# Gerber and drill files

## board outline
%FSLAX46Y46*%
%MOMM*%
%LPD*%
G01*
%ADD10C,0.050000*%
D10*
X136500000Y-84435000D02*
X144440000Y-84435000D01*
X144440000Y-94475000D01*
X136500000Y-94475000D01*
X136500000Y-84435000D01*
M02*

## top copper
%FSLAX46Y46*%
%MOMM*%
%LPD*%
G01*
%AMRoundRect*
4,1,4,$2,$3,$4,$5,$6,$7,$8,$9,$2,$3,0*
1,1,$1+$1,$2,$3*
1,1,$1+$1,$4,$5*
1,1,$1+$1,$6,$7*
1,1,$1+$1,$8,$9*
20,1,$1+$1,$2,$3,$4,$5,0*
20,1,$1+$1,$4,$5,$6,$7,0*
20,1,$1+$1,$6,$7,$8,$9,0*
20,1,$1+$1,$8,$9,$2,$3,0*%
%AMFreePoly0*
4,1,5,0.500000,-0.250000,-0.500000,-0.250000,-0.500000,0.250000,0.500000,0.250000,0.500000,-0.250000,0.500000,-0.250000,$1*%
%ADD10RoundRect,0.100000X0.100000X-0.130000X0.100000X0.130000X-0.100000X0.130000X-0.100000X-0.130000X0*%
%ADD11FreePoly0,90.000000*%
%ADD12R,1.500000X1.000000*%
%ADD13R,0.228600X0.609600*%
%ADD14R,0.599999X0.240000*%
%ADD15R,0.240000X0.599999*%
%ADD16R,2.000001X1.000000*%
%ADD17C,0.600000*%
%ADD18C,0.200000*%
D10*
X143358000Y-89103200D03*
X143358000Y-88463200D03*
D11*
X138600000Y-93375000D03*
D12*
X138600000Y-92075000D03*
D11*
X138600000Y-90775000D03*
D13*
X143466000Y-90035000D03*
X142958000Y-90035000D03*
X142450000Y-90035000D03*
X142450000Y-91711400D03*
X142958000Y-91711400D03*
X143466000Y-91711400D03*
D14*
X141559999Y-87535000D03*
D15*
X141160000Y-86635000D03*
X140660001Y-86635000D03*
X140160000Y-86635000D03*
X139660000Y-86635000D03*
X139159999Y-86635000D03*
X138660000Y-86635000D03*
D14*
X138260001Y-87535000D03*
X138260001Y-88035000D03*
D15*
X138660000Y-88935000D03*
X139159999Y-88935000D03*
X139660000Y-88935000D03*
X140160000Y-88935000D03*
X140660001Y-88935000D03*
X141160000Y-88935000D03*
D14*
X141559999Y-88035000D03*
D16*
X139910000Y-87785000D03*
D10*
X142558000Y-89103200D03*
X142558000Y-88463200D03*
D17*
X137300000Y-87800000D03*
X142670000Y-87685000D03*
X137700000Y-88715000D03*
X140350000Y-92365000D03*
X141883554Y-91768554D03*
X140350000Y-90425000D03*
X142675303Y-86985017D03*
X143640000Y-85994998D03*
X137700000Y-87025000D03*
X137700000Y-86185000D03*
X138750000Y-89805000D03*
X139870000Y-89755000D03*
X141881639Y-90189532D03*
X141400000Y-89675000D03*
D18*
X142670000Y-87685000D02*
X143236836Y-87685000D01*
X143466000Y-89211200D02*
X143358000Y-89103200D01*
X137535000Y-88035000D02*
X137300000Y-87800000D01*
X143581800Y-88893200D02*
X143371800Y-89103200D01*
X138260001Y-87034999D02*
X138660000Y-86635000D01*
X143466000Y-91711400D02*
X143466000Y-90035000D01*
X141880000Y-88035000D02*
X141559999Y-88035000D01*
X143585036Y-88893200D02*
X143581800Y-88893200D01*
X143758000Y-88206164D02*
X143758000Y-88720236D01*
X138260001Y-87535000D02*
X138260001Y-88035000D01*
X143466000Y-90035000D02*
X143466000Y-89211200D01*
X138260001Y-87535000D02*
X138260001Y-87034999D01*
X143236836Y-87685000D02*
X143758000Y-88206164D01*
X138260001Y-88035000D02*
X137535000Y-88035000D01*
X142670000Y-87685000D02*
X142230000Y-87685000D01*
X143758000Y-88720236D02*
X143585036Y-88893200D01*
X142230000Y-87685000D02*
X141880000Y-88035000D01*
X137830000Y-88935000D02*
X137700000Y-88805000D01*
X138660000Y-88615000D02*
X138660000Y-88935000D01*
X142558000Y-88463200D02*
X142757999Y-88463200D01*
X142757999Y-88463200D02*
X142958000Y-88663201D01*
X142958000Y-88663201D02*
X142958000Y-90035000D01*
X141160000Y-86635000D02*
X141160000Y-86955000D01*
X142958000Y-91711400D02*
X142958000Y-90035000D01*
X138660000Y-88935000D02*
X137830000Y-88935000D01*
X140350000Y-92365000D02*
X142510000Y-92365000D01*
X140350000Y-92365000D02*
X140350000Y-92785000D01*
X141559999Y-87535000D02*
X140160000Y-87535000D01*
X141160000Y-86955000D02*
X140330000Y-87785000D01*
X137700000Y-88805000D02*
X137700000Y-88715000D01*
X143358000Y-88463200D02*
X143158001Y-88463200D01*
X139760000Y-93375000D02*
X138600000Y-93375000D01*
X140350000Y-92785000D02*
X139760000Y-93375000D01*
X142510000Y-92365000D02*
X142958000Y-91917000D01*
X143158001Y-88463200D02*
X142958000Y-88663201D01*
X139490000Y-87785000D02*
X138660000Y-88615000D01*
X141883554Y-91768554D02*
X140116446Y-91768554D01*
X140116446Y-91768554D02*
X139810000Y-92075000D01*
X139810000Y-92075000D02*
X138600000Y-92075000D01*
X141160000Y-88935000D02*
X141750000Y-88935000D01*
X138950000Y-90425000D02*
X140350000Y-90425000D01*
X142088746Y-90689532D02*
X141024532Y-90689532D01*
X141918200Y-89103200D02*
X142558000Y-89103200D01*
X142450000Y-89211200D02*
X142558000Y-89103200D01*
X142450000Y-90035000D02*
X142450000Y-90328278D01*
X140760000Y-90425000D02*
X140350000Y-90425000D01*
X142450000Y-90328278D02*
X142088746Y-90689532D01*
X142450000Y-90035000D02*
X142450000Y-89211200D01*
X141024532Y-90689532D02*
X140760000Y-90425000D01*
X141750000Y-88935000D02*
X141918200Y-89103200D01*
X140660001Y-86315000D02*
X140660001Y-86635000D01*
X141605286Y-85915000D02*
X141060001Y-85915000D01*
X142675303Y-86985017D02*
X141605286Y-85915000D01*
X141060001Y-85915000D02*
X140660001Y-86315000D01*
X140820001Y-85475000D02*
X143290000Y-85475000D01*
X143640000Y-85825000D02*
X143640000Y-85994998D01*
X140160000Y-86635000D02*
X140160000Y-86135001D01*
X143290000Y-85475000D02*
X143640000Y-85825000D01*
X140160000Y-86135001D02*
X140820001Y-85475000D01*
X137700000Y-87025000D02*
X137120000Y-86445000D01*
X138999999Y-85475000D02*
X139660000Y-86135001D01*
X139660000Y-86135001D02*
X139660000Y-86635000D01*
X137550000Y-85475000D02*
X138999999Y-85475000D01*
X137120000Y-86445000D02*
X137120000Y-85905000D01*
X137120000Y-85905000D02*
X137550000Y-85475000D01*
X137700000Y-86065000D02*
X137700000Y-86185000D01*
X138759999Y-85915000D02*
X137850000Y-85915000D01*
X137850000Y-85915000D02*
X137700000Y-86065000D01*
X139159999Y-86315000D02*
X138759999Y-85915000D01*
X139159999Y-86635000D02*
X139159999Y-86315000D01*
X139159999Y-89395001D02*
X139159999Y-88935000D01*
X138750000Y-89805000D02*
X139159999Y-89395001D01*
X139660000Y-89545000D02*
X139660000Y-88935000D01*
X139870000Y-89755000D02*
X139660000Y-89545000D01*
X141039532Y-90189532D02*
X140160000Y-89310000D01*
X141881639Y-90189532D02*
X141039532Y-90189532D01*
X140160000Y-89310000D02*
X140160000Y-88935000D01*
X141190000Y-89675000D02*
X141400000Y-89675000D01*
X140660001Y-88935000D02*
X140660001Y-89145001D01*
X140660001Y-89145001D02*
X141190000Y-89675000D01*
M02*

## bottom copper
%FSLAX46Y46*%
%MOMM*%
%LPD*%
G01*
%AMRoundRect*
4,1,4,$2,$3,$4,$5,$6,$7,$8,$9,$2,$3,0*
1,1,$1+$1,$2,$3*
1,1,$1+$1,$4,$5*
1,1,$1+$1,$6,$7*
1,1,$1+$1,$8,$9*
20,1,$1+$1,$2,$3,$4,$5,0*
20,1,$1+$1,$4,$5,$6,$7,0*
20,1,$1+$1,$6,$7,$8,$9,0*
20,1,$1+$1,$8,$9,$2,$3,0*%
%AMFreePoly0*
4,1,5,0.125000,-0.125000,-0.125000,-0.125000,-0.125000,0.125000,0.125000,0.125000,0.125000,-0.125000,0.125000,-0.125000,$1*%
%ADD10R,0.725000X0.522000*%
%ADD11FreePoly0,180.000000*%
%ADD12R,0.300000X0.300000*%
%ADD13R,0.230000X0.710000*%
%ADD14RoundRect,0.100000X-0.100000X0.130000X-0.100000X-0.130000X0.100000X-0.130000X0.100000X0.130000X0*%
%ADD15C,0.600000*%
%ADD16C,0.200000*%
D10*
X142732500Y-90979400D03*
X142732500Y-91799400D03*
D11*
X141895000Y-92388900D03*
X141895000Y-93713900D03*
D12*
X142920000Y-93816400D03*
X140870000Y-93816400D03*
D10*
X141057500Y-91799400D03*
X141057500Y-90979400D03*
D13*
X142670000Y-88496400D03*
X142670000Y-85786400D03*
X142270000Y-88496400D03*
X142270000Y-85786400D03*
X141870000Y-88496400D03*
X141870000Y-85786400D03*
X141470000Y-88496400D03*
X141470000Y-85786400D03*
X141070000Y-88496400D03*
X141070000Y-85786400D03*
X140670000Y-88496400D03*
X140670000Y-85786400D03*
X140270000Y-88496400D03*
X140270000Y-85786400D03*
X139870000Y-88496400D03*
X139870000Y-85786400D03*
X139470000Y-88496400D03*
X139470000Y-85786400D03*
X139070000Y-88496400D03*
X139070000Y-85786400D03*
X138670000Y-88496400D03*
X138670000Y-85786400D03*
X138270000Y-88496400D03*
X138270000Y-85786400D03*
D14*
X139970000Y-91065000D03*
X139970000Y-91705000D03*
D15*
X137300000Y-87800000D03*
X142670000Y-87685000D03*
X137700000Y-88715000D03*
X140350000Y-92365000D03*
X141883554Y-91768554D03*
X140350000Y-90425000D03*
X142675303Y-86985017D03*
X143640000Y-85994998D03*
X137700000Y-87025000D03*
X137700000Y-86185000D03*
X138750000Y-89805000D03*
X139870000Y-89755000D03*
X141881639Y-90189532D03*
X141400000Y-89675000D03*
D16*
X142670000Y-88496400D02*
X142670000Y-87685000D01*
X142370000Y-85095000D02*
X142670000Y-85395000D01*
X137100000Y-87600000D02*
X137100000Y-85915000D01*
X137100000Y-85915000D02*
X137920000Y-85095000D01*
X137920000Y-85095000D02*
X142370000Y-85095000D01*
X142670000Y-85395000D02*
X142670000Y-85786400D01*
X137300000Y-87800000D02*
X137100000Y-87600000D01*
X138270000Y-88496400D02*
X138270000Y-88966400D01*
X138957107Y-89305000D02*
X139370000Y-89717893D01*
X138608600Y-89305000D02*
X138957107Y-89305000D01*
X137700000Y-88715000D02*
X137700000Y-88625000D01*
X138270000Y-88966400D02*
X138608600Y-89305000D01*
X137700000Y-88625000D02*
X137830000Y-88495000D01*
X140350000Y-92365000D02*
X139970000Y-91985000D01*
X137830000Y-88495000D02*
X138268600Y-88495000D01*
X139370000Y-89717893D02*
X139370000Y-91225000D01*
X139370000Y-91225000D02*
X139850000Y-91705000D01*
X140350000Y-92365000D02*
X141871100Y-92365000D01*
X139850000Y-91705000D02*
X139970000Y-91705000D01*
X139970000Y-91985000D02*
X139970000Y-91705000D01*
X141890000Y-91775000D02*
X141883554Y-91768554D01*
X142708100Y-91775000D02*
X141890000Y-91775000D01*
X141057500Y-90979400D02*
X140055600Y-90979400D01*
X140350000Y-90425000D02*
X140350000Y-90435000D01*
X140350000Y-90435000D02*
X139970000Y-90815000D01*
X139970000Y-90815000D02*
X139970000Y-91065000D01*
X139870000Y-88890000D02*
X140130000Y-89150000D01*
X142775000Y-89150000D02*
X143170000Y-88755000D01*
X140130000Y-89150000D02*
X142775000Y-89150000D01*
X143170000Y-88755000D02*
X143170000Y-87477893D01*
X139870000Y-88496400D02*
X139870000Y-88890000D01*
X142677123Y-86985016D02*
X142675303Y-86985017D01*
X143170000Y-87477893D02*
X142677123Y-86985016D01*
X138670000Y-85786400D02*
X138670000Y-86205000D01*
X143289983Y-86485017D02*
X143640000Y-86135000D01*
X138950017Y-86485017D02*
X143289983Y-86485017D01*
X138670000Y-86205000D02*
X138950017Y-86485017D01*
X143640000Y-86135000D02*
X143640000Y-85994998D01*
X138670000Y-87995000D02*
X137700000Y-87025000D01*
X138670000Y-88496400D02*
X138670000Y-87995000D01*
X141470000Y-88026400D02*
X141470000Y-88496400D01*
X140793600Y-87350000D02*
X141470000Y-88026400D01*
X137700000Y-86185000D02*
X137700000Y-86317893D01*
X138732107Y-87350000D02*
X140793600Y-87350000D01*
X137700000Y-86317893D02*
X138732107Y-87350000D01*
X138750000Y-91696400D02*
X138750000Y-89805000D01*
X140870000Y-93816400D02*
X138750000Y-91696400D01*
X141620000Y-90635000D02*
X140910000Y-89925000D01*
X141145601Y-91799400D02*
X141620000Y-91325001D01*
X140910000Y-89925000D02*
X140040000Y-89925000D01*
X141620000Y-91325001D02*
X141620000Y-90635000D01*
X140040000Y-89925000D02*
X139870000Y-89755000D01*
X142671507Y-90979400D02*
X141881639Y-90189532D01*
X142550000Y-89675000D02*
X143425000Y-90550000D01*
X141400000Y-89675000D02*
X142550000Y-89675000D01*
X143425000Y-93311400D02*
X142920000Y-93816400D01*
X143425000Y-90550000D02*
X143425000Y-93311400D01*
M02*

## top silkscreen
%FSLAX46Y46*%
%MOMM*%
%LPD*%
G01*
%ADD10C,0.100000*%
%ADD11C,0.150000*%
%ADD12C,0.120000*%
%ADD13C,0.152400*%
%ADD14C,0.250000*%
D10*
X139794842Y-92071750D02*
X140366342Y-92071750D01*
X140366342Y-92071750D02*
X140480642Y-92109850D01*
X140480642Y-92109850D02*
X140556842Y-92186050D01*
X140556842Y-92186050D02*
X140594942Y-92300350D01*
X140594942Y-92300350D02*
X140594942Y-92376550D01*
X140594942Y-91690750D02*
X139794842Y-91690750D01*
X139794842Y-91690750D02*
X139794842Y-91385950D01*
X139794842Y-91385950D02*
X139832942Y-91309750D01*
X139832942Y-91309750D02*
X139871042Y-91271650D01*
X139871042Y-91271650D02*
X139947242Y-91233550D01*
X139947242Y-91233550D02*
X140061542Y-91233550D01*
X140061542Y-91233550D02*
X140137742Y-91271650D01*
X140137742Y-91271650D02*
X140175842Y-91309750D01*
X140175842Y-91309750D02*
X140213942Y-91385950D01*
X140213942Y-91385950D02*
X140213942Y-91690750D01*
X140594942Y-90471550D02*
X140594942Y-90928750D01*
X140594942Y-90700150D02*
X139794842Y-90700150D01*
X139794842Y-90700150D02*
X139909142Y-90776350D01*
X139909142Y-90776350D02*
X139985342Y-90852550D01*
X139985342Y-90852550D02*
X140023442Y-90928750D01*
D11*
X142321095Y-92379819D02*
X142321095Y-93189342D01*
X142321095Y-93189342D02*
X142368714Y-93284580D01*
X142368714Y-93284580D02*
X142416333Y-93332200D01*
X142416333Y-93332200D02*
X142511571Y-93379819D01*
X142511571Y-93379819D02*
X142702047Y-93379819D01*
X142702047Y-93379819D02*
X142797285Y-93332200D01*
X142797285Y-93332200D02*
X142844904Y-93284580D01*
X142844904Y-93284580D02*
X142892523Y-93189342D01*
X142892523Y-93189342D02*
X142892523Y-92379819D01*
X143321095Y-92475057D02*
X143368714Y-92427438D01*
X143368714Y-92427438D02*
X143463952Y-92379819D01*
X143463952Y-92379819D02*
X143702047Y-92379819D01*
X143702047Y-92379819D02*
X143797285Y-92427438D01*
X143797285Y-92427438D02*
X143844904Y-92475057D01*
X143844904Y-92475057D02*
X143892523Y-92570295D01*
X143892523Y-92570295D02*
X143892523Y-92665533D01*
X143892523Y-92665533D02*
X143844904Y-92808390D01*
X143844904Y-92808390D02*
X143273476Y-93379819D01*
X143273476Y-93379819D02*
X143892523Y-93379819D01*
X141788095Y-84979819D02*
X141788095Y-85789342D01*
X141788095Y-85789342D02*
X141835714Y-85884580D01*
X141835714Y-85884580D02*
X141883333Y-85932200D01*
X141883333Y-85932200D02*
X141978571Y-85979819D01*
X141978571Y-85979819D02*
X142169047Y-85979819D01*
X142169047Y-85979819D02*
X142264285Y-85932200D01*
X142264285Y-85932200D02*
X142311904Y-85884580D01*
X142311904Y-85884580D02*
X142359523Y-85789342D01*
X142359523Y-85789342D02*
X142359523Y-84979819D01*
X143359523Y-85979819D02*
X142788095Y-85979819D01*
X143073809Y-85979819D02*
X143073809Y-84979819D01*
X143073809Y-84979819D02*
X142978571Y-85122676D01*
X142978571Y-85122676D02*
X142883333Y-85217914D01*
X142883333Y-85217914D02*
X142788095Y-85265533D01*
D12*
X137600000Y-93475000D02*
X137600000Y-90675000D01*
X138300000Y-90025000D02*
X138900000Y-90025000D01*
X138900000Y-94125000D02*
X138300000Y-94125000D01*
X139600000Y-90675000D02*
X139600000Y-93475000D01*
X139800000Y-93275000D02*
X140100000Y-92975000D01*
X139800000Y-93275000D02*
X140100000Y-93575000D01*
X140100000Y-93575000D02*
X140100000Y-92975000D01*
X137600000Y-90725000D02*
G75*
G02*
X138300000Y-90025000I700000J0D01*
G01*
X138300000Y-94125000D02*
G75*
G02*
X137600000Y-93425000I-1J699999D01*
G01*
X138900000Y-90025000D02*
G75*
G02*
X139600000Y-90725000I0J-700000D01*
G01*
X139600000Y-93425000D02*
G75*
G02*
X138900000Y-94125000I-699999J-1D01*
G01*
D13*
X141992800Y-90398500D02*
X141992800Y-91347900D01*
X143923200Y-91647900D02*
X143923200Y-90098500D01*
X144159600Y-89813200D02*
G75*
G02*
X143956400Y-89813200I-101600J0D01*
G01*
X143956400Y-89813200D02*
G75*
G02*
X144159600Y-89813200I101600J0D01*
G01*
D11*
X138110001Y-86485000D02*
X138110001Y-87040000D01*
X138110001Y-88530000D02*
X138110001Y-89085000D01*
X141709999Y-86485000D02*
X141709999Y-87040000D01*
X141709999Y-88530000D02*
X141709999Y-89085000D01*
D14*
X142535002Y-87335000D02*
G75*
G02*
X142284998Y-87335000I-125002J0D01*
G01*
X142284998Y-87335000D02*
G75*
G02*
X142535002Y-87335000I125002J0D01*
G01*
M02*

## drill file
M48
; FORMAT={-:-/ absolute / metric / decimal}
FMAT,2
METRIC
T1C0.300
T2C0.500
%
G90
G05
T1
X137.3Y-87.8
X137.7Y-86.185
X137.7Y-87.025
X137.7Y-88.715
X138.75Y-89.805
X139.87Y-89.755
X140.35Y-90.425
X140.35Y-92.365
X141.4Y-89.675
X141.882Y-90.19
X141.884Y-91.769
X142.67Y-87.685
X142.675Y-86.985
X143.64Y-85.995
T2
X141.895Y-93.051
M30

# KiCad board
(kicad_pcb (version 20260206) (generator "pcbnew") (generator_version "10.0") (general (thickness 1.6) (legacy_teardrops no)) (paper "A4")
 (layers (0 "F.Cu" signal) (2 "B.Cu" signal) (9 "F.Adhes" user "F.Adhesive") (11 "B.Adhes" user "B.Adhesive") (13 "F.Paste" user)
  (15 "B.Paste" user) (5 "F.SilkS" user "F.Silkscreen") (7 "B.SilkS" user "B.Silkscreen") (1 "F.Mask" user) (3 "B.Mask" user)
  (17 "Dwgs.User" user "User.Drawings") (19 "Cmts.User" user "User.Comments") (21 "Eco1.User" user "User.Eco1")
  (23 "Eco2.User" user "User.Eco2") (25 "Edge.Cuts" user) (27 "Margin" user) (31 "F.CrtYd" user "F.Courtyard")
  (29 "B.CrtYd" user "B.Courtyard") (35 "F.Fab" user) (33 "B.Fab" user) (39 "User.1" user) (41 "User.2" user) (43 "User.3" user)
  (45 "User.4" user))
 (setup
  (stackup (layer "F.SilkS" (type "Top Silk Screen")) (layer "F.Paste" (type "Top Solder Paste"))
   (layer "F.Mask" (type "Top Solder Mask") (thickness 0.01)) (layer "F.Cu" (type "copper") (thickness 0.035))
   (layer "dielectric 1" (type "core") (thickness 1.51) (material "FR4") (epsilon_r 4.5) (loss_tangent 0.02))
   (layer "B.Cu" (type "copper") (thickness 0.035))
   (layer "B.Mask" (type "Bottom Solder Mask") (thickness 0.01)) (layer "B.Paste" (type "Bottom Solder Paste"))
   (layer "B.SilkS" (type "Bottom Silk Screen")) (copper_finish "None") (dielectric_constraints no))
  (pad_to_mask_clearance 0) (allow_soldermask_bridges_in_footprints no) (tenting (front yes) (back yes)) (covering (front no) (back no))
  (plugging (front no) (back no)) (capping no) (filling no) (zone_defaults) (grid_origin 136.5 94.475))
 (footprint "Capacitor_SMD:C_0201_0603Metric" (layer "F.Cu") (at 143.358 88.7832 90)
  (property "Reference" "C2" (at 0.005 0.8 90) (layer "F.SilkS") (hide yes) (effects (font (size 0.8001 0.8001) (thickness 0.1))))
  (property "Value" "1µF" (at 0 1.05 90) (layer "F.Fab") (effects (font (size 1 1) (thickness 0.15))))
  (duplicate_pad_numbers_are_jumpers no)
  (pad "" smd roundrect (at -0.345 0 90) (size 0.318 0.36) (layers "F.Paste") (roundrect_rratio 0.25))
  (pad "" smd roundrect (at 0.345 0 90) (size 0.318 0.36) (layers "F.Paste") (roundrect_rratio 0.25))
  (pad "1" smd roundrect (at -0.32 0 90) (size 0.46 0.4) (layers "F.Cu" "F.Mask") (roundrect_rratio 0.25) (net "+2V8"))
  (pad "2" smd roundrect (at 0.32 0 90) (size 0.46 0.4) (layers "F.Cu" "F.Mask") (roundrect_rratio 0.25) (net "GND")))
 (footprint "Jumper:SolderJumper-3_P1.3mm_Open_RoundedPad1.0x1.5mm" (layer "F.Cu") (at 138.6 92.075 90)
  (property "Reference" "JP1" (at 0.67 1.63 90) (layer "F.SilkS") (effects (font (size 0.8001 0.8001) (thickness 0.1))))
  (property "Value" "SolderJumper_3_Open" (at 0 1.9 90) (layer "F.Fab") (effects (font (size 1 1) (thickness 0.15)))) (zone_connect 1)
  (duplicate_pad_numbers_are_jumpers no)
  (fp_line (start -1.4 -1) (end 1.4 -1) (stroke (width 0.12) (type solid)) (layer "F.SilkS"))
  (fp_line (start 2.05 -0.3) (end 2.05 0.3) (stroke (width 0.12) (type solid)) (layer "F.SilkS"))
  (fp_line (start -2.05 0.3) (end -2.05 -0.3) (stroke (width 0.12) (type solid)) (layer "F.SilkS"))
  (fp_line (start 1.4 1) (end -1.4 1) (stroke (width 0.12) (type solid)) (layer "F.SilkS"))
  (fp_line (start -1.2 1.2) (end -0.9 1.5) (stroke (width 0.12) (type solid)) (layer "F.SilkS"))
  (fp_line (start -1.2 1.2) (end -1.5 1.5) (stroke (width 0.12) (type solid)) (layer "F.SilkS"))
  (fp_line (start -1.5 1.5) (end -0.9 1.5) (stroke (width 0.12) (type solid)) (layer "F.SilkS"))
  (fp_arc (start 1.35 -1) (mid 1.844975 -0.794975) (end 2.05 -0.3) (stroke (width 0.12) (type solid)) (layer "F.SilkS"))
  (fp_arc (start -2.05 -0.3) (mid -1.844975 -0.794975) (end -1.35 -1) (stroke (width 0.12) (type solid)) (layer "F.SilkS"))
  (fp_arc (start 2.05 0.3) (mid 1.844975 0.794975) (end 1.35 1) (stroke (width 0.12) (type solid)) (layer "F.SilkS"))
  (fp_arc (start -1.35 1) (mid -1.844975 0.794975) (end -2.05 0.3) (stroke (width 0.12) (type solid)) (layer "F.SilkS"))
  (pad "1" smd custom (at -1.3 0 90) (size 1 0.5) (layers "F.Cu" "F.Mask") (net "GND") (zone_connect 2) (thermal_bridge_angle 45)
   (options (clearance outline) (anchor rect)) (primitives))
  (pad "2" smd rect (at 0 0 90) (size 1 1.5) (layers "F.Cu" "F.Mask") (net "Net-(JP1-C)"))
  (pad "3" smd custom (at 1.3 0 90) (size 1 0.5) (layers "F.Cu" "F.Mask") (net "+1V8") (zone_connect 2) (thermal_bridge_angle 45)
   (options (clearance outline) (anchor rect)) (primitives)))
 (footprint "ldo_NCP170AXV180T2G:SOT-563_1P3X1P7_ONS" (layer "F.Cu") (at 142.958 90.8732 -90)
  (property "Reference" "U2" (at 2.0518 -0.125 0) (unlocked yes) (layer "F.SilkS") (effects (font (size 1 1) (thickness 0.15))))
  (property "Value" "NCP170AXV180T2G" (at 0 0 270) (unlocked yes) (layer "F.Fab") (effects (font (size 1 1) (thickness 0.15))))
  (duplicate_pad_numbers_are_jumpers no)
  (fp_line (start -0.4747 0.9652) (end 0.4747 0.9652) (stroke (width 0.1524) (type solid)) (layer "F.SilkS"))
  (fp_line (start 0.7747 -0.9652) (end -0.7747 -0.9652) (stroke (width 0.1524) (type solid)) (layer "F.SilkS"))
  (fp_circle (center -1.06 -1.1) (end -0.9584 -1.1) (stroke (width 0.1524) (type solid)) (fill no) (layer "F.SilkS"))
  (pad "1" smd rect (at -0.8382 -0.508 270) (size 0.6096 0.2286) (layers "F.Cu" "F.Mask" "F.Paste") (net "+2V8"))
  (pad "2" smd rect (at -0.8382 0 270) (size 0.6096 0.2286) (layers "F.Cu" "F.Mask" "F.Paste") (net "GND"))
  (pad "3" smd rect (at -0.8382 0.508 270) (size 0.6096 0.2286) (layers "F.Cu" "F.Mask" "F.Paste") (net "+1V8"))
  (pad "4" smd rect (at 0.8382 0.508 270) (size 0.6096 0.2286) (layers "F.Cu" "F.Mask" "F.Paste") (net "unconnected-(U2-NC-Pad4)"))
  (pad "5" smd rect (at 0.8382 0 270) (size 0.6096 0.2286) (layers "F.Cu" "F.Mask" "F.Paste") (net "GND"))
  (pad "6" smd rect (at 0.8382 -0.508 270) (size 0.6096 0.2286) (layers "F.Cu" "F.Mask" "F.Paste") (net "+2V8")))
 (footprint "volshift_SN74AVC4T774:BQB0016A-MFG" (layer "F.Cu") (at 139.91 87.785 -90)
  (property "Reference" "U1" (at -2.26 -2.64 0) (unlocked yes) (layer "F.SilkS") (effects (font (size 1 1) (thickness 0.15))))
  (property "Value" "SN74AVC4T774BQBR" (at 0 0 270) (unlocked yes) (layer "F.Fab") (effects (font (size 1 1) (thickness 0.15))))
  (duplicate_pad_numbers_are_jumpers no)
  (fp_line (start -1.3 1.799999) (end -0.745 1.799999) (stroke (width 0.15) (type solid)) (layer "F.SilkS"))
  (fp_line (start 0.745 1.799999) (end 1.3 1.799999) (stroke (width 0.15) (type solid)) (layer "F.SilkS"))
  (fp_line (start -1.3 -1.799999) (end -0.745 -1.799999) (stroke (width 0.15) (type solid)) (layer "F.SilkS"))
  (fp_line (start 0.745 -1.799999) (end 1.3 -1.799999) (stroke (width 0.15) (type solid)) (layer "F.SilkS"))
  (fp_circle (center -0.45 -2.5) (end -0.324998 -2.5) (stroke (width 0.25) (type solid)) (fill no) (layer "F.SilkS"))
  (pad "1" smd rect (at -0.25 -1.649999 270) (size 0.24 0.599999) (layers "F.Cu" "F.Mask" "F.Paste") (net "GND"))
  (pad "2" smd rect (at -1.15 -1.25) (size 0.24 0.599999) (layers "F.Cu" "F.Mask" "F.Paste") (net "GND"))
  (pad "3" smd rect (at -1.15 -0.750001) (size 0.24 0.599999) (layers "F.Cu" "F.Mask" "F.Paste") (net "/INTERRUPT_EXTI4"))
  (pad "4" smd rect (at -1.15 -0.25) (size 0.24 0.599999) (layers "F.Cu" "F.Mask" "F.Paste") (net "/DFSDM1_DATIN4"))
  (pad "5" smd rect (at -1.15 0.25) (size 0.24 0.599999) (layers "F.Cu" "F.Mask" "F.Paste") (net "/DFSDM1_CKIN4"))
  (pad "6" smd rect (at -1.15 0.750001) (size 0.24 0.599999) (layers "F.Cu" "F.Mask" "F.Paste") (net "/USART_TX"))
  (pad "7" smd rect (at -1.15 1.25) (size 0.24 0.599999) (layers "F.Cu" "F.Mask" "F.Paste") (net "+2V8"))
  (pad "8" smd rect (at -0.25 1.649999 270) (size 0.24 0.599999) (layers "F.Cu" "F.Mask" "F.Paste") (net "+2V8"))
  (pad "9" smd rect (at 0.25 1.649999 270) (size 0.24 0.599999) (layers "F.Cu" "F.Mask" "F.Paste") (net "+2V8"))
  (pad "10" smd rect (at 1.15 1.25) (size 0.24 0.599999) (layers "F.Cu" "F.Mask" "F.Paste") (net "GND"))
  (pad "11" smd rect (at 1.15 0.750001) (size 0.24 0.599999) (layers "F.Cu" "F.Mask" "F.Paste") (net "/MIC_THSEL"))
  (pad "12" smd rect (at 1.15 0.25) (size 0.24 0.599999) (layers "F.Cu" "F.Mask" "F.Paste") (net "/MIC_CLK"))
  (pad "13" smd rect (at 1.15 -0.25) (size 0.24 0.599999) (layers "F.Cu" "F.Mask" "F.Paste") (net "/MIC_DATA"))
  (pad "14" smd rect (at 1.15 -0.750001) (size 0.24 0.599999) (layers "F.Cu" "F.Mask" "F.Paste") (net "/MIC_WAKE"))
  (pad "15" smd rect (at 1.15 -1.25) (size 0.24 0.599999) (layers "F.Cu" "F.Mask" "F.Paste") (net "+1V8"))
  (pad "16" smd rect (at 0.25 -1.649999 270) (size 0.24 0.599999) (layers "F.Cu" "F.Mask" "F.Paste") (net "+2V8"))
  (pad "17" smd rect (at 0 0 270) (size 1 2.000001) (layers "F.Cu" "F.Mask") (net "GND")))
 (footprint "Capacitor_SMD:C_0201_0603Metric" (layer "F.Cu") (at 142.558 88.7832 90)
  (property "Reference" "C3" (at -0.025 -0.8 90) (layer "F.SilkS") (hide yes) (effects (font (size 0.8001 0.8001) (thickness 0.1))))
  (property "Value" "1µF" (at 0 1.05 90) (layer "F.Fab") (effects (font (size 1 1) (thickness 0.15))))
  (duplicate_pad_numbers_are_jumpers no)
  (pad "" smd roundrect (at -0.345 0 90) (size 0.318 0.36) (layers "F.Paste") (roundrect_rratio 0.25))
  (pad "" smd roundrect (at 0.345 0 90) (size 0.318 0.36) (layers "F.Paste") (roundrect_rratio 0.25))
  (pad "1" smd roundrect (at -0.32 0 90) (size 0.46 0.4) (layers "F.Cu" "F.Mask") (roundrect_rratio 0.25) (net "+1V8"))
  (pad "2" smd roundrect (at 0.32 0 90) (size 0.46 0.4) (layers "F.Cu" "F.Mask") (roundrect_rratio 0.25) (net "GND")))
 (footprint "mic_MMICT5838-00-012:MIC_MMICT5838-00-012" (layer "B.Cu") (at 141.895 92.3414 180)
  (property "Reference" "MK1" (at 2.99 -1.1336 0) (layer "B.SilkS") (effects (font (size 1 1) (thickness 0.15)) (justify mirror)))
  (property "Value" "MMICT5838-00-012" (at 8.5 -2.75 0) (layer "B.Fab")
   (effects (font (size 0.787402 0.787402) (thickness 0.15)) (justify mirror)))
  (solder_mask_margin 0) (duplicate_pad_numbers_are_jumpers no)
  (pad "" np_thru_hole circle (at 0 -0.71 180) (size 0.5 0.5) (drill 0.5) (layers "*.Cu" "*.Mask"))
  (pad "1" smd rect (at -0.8375 1.362 180) (size 0.725 0.522) (layers "B.Cu") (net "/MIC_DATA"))
  (pad "2" smd rect (at -0.8375 0.542 180) (size 0.725 0.522) (layers "B.Cu") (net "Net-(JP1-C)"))
  (pad "3_1" smd custom (at 0 -0.0475 180) (size 0.25 0.25) (layers "B.Cu") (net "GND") (options (clearance outline) (anchor rect))
   (primitives))
  (pad "3_2" smd custom (at 0 -1.3725 180) (size 0.25 0.25) (layers "B.Cu") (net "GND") (options (clearance outline) (anchor rect))
   (primitives))
  (pad "4" smd rect (at -1.025 -1.475 180) (size 0.3 0.3) (layers "B.Cu") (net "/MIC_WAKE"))
  (pad "5" smd rect (at 1.025 -1.475 180) (size 0.3 0.3) (layers "B.Cu") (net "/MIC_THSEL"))
  (pad "6" smd rect (at 0.8375 0.542 180) (size 0.725 0.522) (layers "B.Cu") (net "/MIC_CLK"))
  (pad "7" smd rect (at 0.8375 1.362 180) (size 0.725 0.522) (layers "B.Cu") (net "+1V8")))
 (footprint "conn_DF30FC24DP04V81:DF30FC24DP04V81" (layer "B.Cu") (at 140.47 87.1414 180)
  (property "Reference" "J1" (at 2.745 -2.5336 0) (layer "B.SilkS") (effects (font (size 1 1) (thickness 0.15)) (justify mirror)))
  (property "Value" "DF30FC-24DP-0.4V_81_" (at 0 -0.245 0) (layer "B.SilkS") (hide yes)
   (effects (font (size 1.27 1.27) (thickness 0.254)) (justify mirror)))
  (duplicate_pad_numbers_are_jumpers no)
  (pad "1" smd rect (at -2.2 -1.355 180) (size 0.23 0.71) (layers "B.Cu" "B.Mask" "B.Paste") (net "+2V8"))
  (pad "2" smd rect (at -2.2 1.355 180) (size 0.23 0.71) (layers "B.Cu" "B.Mask" "B.Paste") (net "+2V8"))
  (pad "3" smd rect (at -1.8 -1.355 180) (size 0.23 0.71) (layers "B.Cu" "B.Mask" "B.Paste") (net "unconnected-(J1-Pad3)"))
  (pad "4" smd rect (at -1.8 1.355 180) (size 0.23 0.71) (layers "B.Cu" "B.Mask" "B.Paste") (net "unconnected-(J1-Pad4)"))
  (pad "5" smd rect (at -1.4 -1.355 180) (size 0.23 0.71) (layers "B.Cu" "B.Mask" "B.Paste") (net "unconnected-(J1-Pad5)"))
  (pad "6" smd rect (at -1.4 1.355 180) (size 0.23 0.71) (layers "B.Cu" "B.Mask" "B.Paste") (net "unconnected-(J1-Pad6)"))
  (pad "7" smd rect (at -1 -1.355 180) (size 0.23 0.71) (layers "B.Cu" "B.Mask" "B.Paste") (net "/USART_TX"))
  (pad "8" smd rect (at -1 1.355 180) (size 0.23 0.71) (layers "B.Cu" "B.Mask" "B.Paste") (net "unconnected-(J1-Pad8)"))
  (pad "9" smd rect (at -0.6 -1.355 180) (size 0.23 0.71) (layers "B.Cu" "B.Mask" "B.Paste") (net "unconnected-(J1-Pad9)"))
  (pad "10" smd rect (at -0.6 1.355 180) (size 0.23 0.71) (layers "B.Cu" "B.Mask" "B.Paste") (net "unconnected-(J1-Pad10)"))
  (pad "11" smd rect (at -0.2 -1.355 180) (size 0.23 0.71) (layers "B.Cu" "B.Mask" "B.Paste") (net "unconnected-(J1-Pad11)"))
  (pad "12" smd rect (at -0.2 1.355 180) (size 0.23 0.71) (layers "B.Cu" "B.Mask" "B.Paste") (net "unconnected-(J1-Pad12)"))
  (pad "13" smd rect (at 0.2 -1.355 180) (size 0.23 0.71) (layers "B.Cu" "B.Mask" "B.Paste") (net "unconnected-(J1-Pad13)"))
  (pad "14" smd rect (at 0.2 1.355 180) (size 0.23 0.71) (layers "B.Cu" "B.Mask" "B.Paste") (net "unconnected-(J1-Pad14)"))
  (pad "15" smd rect (at 0.6 -1.355 180) (size 0.23 0.71) (layers "B.Cu" "B.Mask" "B.Paste") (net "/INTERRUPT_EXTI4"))
  (pad "16" smd rect (at 0.6 1.355 180) (size 0.23 0.71) (layers "B.Cu" "B.Mask" "B.Paste") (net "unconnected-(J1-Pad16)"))
  (pad "17" smd rect (at 1 -1.355 180) (size 0.23 0.71) (layers "B.Cu" "B.Mask" "B.Paste") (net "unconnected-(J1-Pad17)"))
  (pad "18" smd rect (at 1 1.355 180) (size 0.23 0.71) (layers "B.Cu" "B.Mask" "B.Paste") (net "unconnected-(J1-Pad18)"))
  (pad "19" smd rect (at 1.4 -1.355 180) (size 0.23 0.71) (layers "B.Cu" "B.Mask" "B.Paste") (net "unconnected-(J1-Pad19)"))
  (pad "20" smd rect (at 1.4 1.355 180) (size 0.23 0.71) (layers "B.Cu" "B.Mask" "B.Paste") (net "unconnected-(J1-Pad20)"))
  (pad "21" smd rect (at 1.8 -1.355 180) (size 0.23 0.71) (layers "B.Cu" "B.Mask" "B.Paste") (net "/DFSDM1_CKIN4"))
  (pad "22" smd rect (at 1.8 1.355 180) (size 0.23 0.71) (layers "B.Cu" "B.Mask" "B.Paste") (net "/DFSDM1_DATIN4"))
  (pad "23" smd rect (at 2.2 -1.355 180) (size 0.23 0.71) (layers "B.Cu" "B.Mask" "B.Paste") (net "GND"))
  (pad "24" smd rect (at 2.2 1.355 180) (size 0.23 0.71) (layers "B.Cu" "B.Mask" "B.Paste") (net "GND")))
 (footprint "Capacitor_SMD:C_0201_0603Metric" (layer "B.Cu") (at 139.97 91.385 -90)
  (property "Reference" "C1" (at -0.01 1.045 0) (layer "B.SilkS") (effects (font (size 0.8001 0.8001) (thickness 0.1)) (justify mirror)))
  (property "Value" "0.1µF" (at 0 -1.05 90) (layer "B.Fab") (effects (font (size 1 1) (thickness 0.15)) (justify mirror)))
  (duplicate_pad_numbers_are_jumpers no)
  (pad "" smd roundrect (at -0.345 0 270) (size 0.318 0.36) (layers "B.Paste") (roundrect_rratio 0.25))
  (pad "" smd roundrect (at 0.345 0 270) (size 0.318 0.36) (layers "B.Paste") (roundrect_rratio 0.25))
  (pad "1" smd roundrect (at -0.32 0 270) (size 0.46 0.4) (layers "B.Cu" "B.Mask") (roundrect_rratio 0.25) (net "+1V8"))
  (pad "2" smd roundrect (at 0.32 0 270) (size 0.46 0.4) (layers "B.Cu" "B.Mask") (roundrect_rratio 0.25) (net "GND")))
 (gr_rect (start 136.5 84.435) (end 144.44 94.475) (stroke (width 0.05) (type default)) (fill no) (layer "Edge.Cuts"))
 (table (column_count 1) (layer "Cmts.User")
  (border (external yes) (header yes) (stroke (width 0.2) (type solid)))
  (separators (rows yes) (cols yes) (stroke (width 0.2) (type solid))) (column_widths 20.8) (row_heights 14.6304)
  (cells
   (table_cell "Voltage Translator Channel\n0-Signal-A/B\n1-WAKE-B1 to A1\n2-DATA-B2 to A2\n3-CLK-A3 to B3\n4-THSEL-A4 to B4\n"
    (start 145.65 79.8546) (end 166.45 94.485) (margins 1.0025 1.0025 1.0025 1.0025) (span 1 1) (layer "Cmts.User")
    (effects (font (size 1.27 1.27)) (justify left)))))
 (segment (start 142.67 87.685) (end 143.236836 87.685) (width 0.2) (layer "F.Cu") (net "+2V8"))
 (segment (start 143.466 89.2112) (end 143.358 89.1032) (width 0.2) (layer "F.Cu") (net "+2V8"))
 (segment (start 137.535 88.035) (end 137.3 87.8) (width 0.2) (layer "F.Cu") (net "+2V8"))
 (segment (start 143.5818 88.8932) (end 143.3718 89.1032) (width 0.2) (layer "F.Cu") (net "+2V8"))
 (segment (start 138.260001 87.034999) (end 138.66 86.635) (width 0.2) (layer "F.Cu") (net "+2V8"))
 (segment (start 143.466 91.7114) (end 143.466 90.035) (width 0.2) (layer "F.Cu") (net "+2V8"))
 (segment (start 141.88 88.035) (end 141.559999 88.035) (width 0.2) (layer "F.Cu") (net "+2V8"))
 (segment (start 143.585036 88.8932) (end 143.5818 88.8932) (width 0.2) (layer "F.Cu") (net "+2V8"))
 (segment (start 143.758 88.206164) (end 143.758 88.720236) (width 0.2) (layer "F.Cu") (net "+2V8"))
 (segment (start 138.260001 87.535) (end 138.260001 88.035) (width 0.2) (layer "F.Cu") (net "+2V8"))
 (segment (start 143.466 90.035) (end 143.466 89.2112) (width 0.2) (layer "F.Cu") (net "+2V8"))
 (segment (start 138.260001 87.535) (end 138.260001 87.034999) (width 0.2) (layer "F.Cu") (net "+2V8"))
 (segment (start 143.236836 87.685) (end 143.758 88.206164) (width 0.2) (layer "F.Cu") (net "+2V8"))
 (segment (start 138.260001 88.035) (end 137.535 88.035) (width 0.2) (layer "F.Cu") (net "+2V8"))
 (segment (start 142.67 87.685) (end 142.23 87.685) (width 0.2) (layer "F.Cu") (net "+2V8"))
 (segment (start 143.758 88.720236) (end 143.585036 88.8932) (width 0.2) (layer "F.Cu") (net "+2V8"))
 (segment (start 142.23 87.685) (end 141.88 88.035) (width 0.2) (layer "F.Cu") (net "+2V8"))
 (via (at 137.3 87.8) (size 0.6) (drill 0.3) (layers "F.Cu" "B.Cu") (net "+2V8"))
 (via (at 142.67 87.685) (size 0.6) (drill 0.3) (layers "F.Cu" "B.Cu") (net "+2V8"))
 (segment (start 142.67 88.4964) (end 142.67 87.685) (width 0.2) (layer "B.Cu") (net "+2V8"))
 (segment (start 142.37 85.095) (end 142.67 85.395) (width 0.2) (layer "B.Cu") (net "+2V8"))
 (segment (start 137.1 87.6) (end 137.1 85.915) (width 0.2) (layer "B.Cu") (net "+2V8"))
 (segment (start 137.1 85.915) (end 137.92 85.095) (width 0.2) (layer "B.Cu") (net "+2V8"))
 (segment (start 137.92 85.095) (end 142.37 85.095) (width 0.2) (layer "B.Cu") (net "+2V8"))
 (segment (start 142.67 85.395) (end 142.67 85.7864) (width 0.2) (layer "B.Cu") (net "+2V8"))
 (segment (start 137.3 87.8) (end 137.1 87.6) (width 0.2) (layer "B.Cu") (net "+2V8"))
 (segment (start 137.83 88.935) (end 137.7 88.805) (width 0.2) (layer "F.Cu") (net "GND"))
 (segment (start 138.66 88.615) (end 138.66 88.935) (width 0.2) (layer "F.Cu") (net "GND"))
 (segment (start 142.558 88.4632) (end 142.757999 88.4632) (width 0.2) (layer "F.Cu") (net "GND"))
 (segment (start 142.757999 88.4632) (end 142.958 88.663201) (width 0.2) (layer "F.Cu") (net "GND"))
 (segment (start 142.958 88.663201) (end 142.958 90.035) (width 0.2) (layer "F.Cu") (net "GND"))
 (segment (start 141.16 86.635) (end 141.16 86.955) (width 0.2) (layer "F.Cu") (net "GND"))
 (segment (start 142.958 91.7114) (end 142.958 90.035) (width 0.2) (layer "F.Cu") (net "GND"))
 (segment (start 138.66 88.935) (end 137.83 88.935) (width 0.2) (layer "F.Cu") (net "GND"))
 (segment (start 140.35 92.365) (end 142.51 92.365) (width 0.2) (layer "F.Cu") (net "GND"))
 (segment (start 140.35 92.365) (end 140.35 92.785) (width 0.2) (layer "F.Cu") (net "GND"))
 (segment (start 141.559999 87.535) (end 140.16 87.535) (width 0.2) (layer "F.Cu") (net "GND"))
 (segment (start 141.16 86.955) (end 140.33 87.785) (width 0.2) (layer "F.Cu") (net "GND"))
 (segment (start 137.7 88.805) (end 137.7 88.715) (width 0.2) (layer "F.Cu") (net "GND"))
 (segment (start 143.358 88.4632) (end 143.158001 88.4632) (width 0.2) (layer "F.Cu") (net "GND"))
 (segment (start 139.76 93.375) (end 138.6 93.375) (width 0.2) (layer "F.Cu") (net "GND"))
 (segment (start 140.35 92.785) (end 139.76 93.375) (width 0.2) (layer "F.Cu") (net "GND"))
 (segment (start 142.51 92.365) (end 142.958 91.917) (width 0.2) (layer "F.Cu") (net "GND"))
 (segment (start 143.158001 88.4632) (end 142.958 88.663201) (width 0.2) (layer "F.Cu") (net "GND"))
 (segment (start 139.49 87.785) (end 138.66 88.615) (width 0.2) (layer "F.Cu") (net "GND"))
 (via (at 137.7 88.715) (size 0.6) (drill 0.3) (layers "F.Cu" "B.Cu") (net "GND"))
 (via (at 140.35 92.365) (size 0.6) (drill 0.3) (layers "F.Cu" "B.Cu") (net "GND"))
 (segment (start 138.27 88.4964) (end 138.27 88.9664) (width 0.2) (layer "B.Cu") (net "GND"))
 (segment (start 138.957107 89.305) (end 139.37 89.717893) (width 0.2) (layer "B.Cu") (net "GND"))
 (segment (start 138.6086 89.305) (end 138.957107 89.305) (width 0.2) (layer "B.Cu") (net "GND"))
 (segment (start 137.7 88.715) (end 137.7 88.625) (width 0.2) (layer "B.Cu") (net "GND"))
 (segment (start 138.27 88.9664) (end 138.6086 89.305) (width 0.2) (layer "B.Cu") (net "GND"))
 (segment (start 137.7 88.625) (end 137.83 88.495) (width 0.2) (layer "B.Cu") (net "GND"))
 (segment (start 140.35 92.365) (end 139.97 91.985) (width 0.2) (layer "B.Cu") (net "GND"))
 (segment (start 137.83 88.495) (end 138.2686 88.495) (width 0.2) (layer "B.Cu") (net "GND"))
 (segment (start 139.37 89.717893) (end 139.37 91.225) (width 0.2) (layer "B.Cu") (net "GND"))
 (segment (start 139.37 91.225) (end 139.85 91.705) (width 0.2) (layer "B.Cu") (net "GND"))
 (segment (start 140.35 92.365) (end 141.8711 92.365) (width 0.2) (layer "B.Cu") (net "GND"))
 (segment (start 139.85 91.705) (end 139.97 91.705) (width 0.2) (layer "B.Cu") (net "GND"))
 (segment (start 139.97 91.985) (end 139.97 91.705) (width 0.2) (layer "B.Cu") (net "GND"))
 (segment (start 141.883554 91.768554) (end 140.116446 91.768554) (width 0.2) (layer "F.Cu") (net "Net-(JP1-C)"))
 (segment (start 140.116446 91.768554) (end 139.81 92.075) (width 0.2) (layer "F.Cu") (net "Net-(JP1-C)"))
 (segment (start 139.81 92.075) (end 138.6 92.075) (width 0.2) (layer "F.Cu") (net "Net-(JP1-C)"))
 (via (at 141.883554 91.768554) (size 0.6) (drill 0.3) (layers "F.Cu" "B.Cu") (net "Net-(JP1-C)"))
 (segment (start 141.89 91.775) (end 141.883554 91.768554) (width 0.2) (layer "B.Cu") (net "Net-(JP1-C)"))
 (segment (start 142.7081 91.775) (end 141.89 91.775) (width 0.2) (layer "B.Cu") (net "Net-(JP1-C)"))
 (segment (start 141.16 88.935) (end 141.75 88.935) (width 0.2) (layer "F.Cu") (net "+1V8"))
 (segment (start 138.95 90.425) (end 140.35 90.425) (width 0.2) (layer "F.Cu") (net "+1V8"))
 (segment (start 142.088746 90.689532) (end 141.024532 90.689532) (width 0.2) (layer "F.Cu") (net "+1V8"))
 (segment (start 141.9182 89.1032) (end 142.558 89.1032) (width 0.2) (layer "F.Cu") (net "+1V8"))
 (segment (start 142.45 89.2112) (end 142.558 89.1032) (width 0.2) (layer "F.Cu") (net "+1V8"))
 (segment (start 142.45 90.035) (end 142.45 90.328278) (width 0.2) (layer "F.Cu") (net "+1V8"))
 (segment (start 140.76 90.425) (end 140.35 90.425) (width 0.2) (layer "F.Cu") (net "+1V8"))
 (segment (start 142.45 90.328278) (end 142.088746 90.689532) (width 0.2) (layer "F.Cu") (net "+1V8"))
 (segment (start 142.45 90.035) (end 142.45 89.2112) (width 0.2) (layer "F.Cu") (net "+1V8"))
 (segment (start 141.024532 90.689532) (end 140.76 90.425) (width 0.2) (layer "F.Cu") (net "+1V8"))
 (segment (start 141.75 88.935) (end 141.9182 89.1032) (width 0.2) (layer "F.Cu") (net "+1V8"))
 (via (at 140.35 90.425) (size 0.6) (drill 0.3) (layers "F.Cu" "B.Cu") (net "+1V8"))
 (segment (start 141.0575 90.9794) (end 140.0556 90.9794) (width 0.2) (layer "B.Cu") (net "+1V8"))
 (segment (start 140.35 90.425) (end 140.35 90.435) (width 0.2) (layer "B.Cu") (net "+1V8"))
 (segment (start 140.35 90.435) (end 139.97 90.815) (width 0.2) (layer "B.Cu") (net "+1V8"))
 (segment (start 139.97 90.815) (end 139.97 91.065) (width 0.2) (layer "B.Cu") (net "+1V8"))
 (segment (start 140.660001 86.315) (end 140.660001 86.635) (width 0.2) (layer "F.Cu") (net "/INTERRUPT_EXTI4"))
 (segment (start 141.605286 85.915) (end 141.060001 85.915) (width 0.2) (layer "F.Cu") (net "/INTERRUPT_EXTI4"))
 (segment (start 142.675303 86.985017) (end 141.605286 85.915) (width 0.2) (layer "F.Cu") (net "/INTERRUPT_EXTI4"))
 (segment (start 141.060001 85.915) (end 140.660001 86.315) (width 0.2) (layer "F.Cu") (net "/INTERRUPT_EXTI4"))
 (via (at 142.675303 86.985017) (size 0.6) (drill 0.3) (layers "F.Cu" "B.Cu") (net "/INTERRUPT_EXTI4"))
 (segment (start 139.87 88.89) (end 140.13 89.15) (width 0.2) (layer "B.Cu") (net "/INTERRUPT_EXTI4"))
 (segment (start 142.775 89.15) (end 143.17 88.755) (width 0.2) (layer "B.Cu") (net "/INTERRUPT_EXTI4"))
 (segment (start 140.13 89.15) (end 142.775 89.15) (width 0.2) (layer "B.Cu") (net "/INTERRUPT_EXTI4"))
 (segment (start 143.17 88.755) (end 143.17 87.477893) (width 0.2) (layer "B.Cu") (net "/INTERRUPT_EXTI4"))
 (segment (start 139.87 88.4964) (end 139.87 88.89) (width 0.2) (layer "B.Cu") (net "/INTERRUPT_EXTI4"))
 (segment (start 142.677123 86.985016) (end 142.675303 86.985017) (width 0.2) (layer "B.Cu") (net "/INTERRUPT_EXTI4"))
 (segment (start 143.17 87.477893) (end 142.677123 86.985016) (width 0.2) (layer "B.Cu") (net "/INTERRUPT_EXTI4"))
 (segment (start 140.820001 85.475) (end 143.29 85.475) (width 0.2) (layer "F.Cu") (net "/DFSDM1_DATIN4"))
 (segment (start 143.64 85.825) (end 143.64 85.994998) (width 0.2) (layer "F.Cu") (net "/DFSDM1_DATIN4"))
 (segment (start 140.16 86.635) (end 140.16 86.135001) (width 0.2) (layer "F.Cu") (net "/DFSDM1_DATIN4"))
 (segment (start 143.29 85.475) (end 143.64 85.825) (width 0.2) (layer "F.Cu") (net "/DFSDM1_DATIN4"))
 (segment (start 140.16 86.135001) (end 140.820001 85.475) (width 0.2) (layer "F.Cu") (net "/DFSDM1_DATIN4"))
 (via (at 143.64 85.994998) (size 0.6) (drill 0.3) (layers "F.Cu" "B.Cu") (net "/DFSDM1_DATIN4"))
 (segment (start 138.67 85.7864) (end 138.67 86.205) (width 0.2) (layer "B.Cu") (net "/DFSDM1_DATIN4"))
 (segment (start 143.289983 86.485017) (end 143.64 86.135) (width 0.2) (layer "B.Cu") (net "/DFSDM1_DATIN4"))
 (segment (start 138.950017 86.485017) (end 143.289983 86.485017) (width 0.2) (layer "B.Cu") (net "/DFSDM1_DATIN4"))
 (segment (start 138.67 86.205) (end 138.950017 86.485017) (width 0.2) (layer "B.Cu") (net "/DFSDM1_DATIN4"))
 (segment (start 143.64 86.135) (end 143.64 85.994998) (width 0.2) (layer "B.Cu") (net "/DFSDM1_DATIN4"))
 (segment (start 137.7 87.025) (end 137.12 86.445) (width 0.2) (layer "F.Cu") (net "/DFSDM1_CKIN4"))
 (segment (start 138.999999 85.475) (end 139.66 86.135001) (width 0.2) (layer "F.Cu") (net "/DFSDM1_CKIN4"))
 (segment (start 139.66 86.135001) (end 139.66 86.635) (width 0.2) (layer "F.Cu") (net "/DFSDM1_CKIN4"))
 (segment (start 137.55 85.475) (end 138.999999 85.475) (width 0.2) (layer "F.Cu") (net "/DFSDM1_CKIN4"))
 (segment (start 137.12 86.445) (end 137.12 85.905) (width 0.2) (layer "F.Cu") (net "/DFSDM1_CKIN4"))
 (segment (start 137.12 85.905) (end 137.55 85.475) (width 0.2) (layer "F.Cu") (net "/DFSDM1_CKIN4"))
 (via (at 137.7 87.025) (size 0.6) (drill 0.3) (layers "F.Cu" "B.Cu") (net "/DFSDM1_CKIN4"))
 (segment (start 138.67 87.995) (end 137.7 87.025) (width 0.2) (layer "B.Cu") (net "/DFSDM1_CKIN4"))
 (segment (start 138.67 88.4964) (end 138.67 87.995) (width 0.2) (layer "B.Cu") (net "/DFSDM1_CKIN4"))
 (segment (start 137.7 86.065) (end 137.7 86.185) (width 0.2) (layer "F.Cu") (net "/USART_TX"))
 (segment (start 138.759999 85.915) (end 137.85 85.915) (width 0.2) (layer "F.Cu") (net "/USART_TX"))
 (segment (start 137.85 85.915) (end 137.7 86.065) (width 0.2) (layer "F.Cu") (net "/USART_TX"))
 (segment (start 139.159999 86.315) (end 138.759999 85.915) (width 0.2) (layer "F.Cu") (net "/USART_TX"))
 (segment (start 139.159999 86.635) (end 139.159999 86.315) (width 0.2) (layer "F.Cu") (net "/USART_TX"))
 (via (at 137.7 86.185) (size 0.6) (drill 0.3) (layers "F.Cu" "B.Cu") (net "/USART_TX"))
 (segment (start 141.47 88.0264) (end 141.47 88.4964) (width 0.2) (layer "B.Cu") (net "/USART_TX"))
 (segment (start 140.7936 87.35) (end 141.47 88.0264) (width 0.2) (layer "B.Cu") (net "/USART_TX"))
 (segment (start 137.7 86.185) (end 137.7 86.317893) (width 0.2) (layer "B.Cu") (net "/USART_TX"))
 (segment (start 138.732107 87.35) (end 140.7936 87.35) (width 0.2) (layer "B.Cu") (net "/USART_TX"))
 (segment (start 137.7 86.317893) (end 138.732107 87.35) (width 0.2) (layer "B.Cu") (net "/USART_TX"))
 (segment (start 139.159999 89.395001) (end 139.159999 88.935) (width 0.2) (layer "F.Cu") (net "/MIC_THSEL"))
 (segment (start 138.75 89.805) (end 139.159999 89.395001) (width 0.2) (layer "F.Cu") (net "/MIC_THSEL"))
 (via (at 138.75 89.805) (size 0.6) (drill 0.3) (layers "F.Cu" "B.Cu") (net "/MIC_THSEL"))
 (segment (start 138.75 91.6964) (end 138.75 89.805) (width 0.2) (layer "B.Cu") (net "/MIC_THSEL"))
 (segment (start 140.87 93.8164) (end 138.75 91.6964) (width 0.2) (layer "B.Cu") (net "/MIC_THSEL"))
 (segment (start 139.66 89.545) (end 139.66 88.935) (width 0.2) (layer "F.Cu") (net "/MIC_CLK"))
 (segment (start 139.87 89.755) (end 139.66 89.545) (width 0.2) (layer "F.Cu") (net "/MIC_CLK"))
 (via (at 139.87 89.755) (size 0.6) (drill 0.3) (layers "F.Cu" "B.Cu") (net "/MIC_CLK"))
 (segment (start 141.62 90.635) (end 140.91 89.925) (width 0.2) (layer "B.Cu") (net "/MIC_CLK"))
 (segment (start 141.145601 91.7994) (end 141.62 91.325001) (width 0.2) (layer "B.Cu") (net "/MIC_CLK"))
 (segment (start 140.91 89.925) (end 140.04 89.925) (width 0.2) (layer "B.Cu") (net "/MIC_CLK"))
 (segment (start 141.62 91.325001) (end 141.62 90.635) (width 0.2) (layer "B.Cu") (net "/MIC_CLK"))
 (segment (start 140.04 89.925) (end 139.87 89.755) (width 0.2) (layer "B.Cu") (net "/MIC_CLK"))
 (segment (start 141.039532 90.189532) (end 140.16 89.31) (width 0.2) (layer "F.Cu") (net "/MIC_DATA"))
 (segment (start 141.881639 90.189532) (end 141.039532 90.189532) (width 0.2) (layer "F.Cu") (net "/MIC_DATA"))
 (segment (start 140.16 89.31) (end 140.16 88.935) (width 0.2) (layer "F.Cu") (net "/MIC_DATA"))
 (via (at 141.881639 90.189532) (size 0.6) (drill 0.3) (layers "F.Cu" "B.Cu") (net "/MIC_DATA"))
 (segment (start 142.671507 90.9794) (end 141.881639 90.189532) (width 0.2) (layer "B.Cu") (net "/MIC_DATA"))
 (segment (start 141.19 89.675) (end 141.4 89.675) (width 0.2) (layer "F.Cu") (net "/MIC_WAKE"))
 (segment (start 140.660001 88.935) (end 140.660001 89.145001) (width 0.2) (layer "F.Cu") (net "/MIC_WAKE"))
 (segment (start 140.660001 89.145001) (end 141.19 89.675) (width 0.2) (layer "F.Cu") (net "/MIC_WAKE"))
 (via (at 141.4 89.675) (size 0.6) (drill 0.3) (layers "F.Cu" "B.Cu") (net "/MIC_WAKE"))
 (segment (start 142.55 89.675) (end 143.425 90.55) (width 0.2) (layer "B.Cu") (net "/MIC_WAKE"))
 (segment (start 141.4 89.675) (end 142.55 89.675) (width 0.2) (layer "B.Cu") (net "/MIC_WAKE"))
 (segment (start 143.425 93.3114) (end 142.92 93.8164) (width 0.2) (layer "B.Cu") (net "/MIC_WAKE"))
 (segment (start 143.425 90.55) (end 143.425 93.3114) (width 0.2) (layer "B.Cu") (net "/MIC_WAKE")))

